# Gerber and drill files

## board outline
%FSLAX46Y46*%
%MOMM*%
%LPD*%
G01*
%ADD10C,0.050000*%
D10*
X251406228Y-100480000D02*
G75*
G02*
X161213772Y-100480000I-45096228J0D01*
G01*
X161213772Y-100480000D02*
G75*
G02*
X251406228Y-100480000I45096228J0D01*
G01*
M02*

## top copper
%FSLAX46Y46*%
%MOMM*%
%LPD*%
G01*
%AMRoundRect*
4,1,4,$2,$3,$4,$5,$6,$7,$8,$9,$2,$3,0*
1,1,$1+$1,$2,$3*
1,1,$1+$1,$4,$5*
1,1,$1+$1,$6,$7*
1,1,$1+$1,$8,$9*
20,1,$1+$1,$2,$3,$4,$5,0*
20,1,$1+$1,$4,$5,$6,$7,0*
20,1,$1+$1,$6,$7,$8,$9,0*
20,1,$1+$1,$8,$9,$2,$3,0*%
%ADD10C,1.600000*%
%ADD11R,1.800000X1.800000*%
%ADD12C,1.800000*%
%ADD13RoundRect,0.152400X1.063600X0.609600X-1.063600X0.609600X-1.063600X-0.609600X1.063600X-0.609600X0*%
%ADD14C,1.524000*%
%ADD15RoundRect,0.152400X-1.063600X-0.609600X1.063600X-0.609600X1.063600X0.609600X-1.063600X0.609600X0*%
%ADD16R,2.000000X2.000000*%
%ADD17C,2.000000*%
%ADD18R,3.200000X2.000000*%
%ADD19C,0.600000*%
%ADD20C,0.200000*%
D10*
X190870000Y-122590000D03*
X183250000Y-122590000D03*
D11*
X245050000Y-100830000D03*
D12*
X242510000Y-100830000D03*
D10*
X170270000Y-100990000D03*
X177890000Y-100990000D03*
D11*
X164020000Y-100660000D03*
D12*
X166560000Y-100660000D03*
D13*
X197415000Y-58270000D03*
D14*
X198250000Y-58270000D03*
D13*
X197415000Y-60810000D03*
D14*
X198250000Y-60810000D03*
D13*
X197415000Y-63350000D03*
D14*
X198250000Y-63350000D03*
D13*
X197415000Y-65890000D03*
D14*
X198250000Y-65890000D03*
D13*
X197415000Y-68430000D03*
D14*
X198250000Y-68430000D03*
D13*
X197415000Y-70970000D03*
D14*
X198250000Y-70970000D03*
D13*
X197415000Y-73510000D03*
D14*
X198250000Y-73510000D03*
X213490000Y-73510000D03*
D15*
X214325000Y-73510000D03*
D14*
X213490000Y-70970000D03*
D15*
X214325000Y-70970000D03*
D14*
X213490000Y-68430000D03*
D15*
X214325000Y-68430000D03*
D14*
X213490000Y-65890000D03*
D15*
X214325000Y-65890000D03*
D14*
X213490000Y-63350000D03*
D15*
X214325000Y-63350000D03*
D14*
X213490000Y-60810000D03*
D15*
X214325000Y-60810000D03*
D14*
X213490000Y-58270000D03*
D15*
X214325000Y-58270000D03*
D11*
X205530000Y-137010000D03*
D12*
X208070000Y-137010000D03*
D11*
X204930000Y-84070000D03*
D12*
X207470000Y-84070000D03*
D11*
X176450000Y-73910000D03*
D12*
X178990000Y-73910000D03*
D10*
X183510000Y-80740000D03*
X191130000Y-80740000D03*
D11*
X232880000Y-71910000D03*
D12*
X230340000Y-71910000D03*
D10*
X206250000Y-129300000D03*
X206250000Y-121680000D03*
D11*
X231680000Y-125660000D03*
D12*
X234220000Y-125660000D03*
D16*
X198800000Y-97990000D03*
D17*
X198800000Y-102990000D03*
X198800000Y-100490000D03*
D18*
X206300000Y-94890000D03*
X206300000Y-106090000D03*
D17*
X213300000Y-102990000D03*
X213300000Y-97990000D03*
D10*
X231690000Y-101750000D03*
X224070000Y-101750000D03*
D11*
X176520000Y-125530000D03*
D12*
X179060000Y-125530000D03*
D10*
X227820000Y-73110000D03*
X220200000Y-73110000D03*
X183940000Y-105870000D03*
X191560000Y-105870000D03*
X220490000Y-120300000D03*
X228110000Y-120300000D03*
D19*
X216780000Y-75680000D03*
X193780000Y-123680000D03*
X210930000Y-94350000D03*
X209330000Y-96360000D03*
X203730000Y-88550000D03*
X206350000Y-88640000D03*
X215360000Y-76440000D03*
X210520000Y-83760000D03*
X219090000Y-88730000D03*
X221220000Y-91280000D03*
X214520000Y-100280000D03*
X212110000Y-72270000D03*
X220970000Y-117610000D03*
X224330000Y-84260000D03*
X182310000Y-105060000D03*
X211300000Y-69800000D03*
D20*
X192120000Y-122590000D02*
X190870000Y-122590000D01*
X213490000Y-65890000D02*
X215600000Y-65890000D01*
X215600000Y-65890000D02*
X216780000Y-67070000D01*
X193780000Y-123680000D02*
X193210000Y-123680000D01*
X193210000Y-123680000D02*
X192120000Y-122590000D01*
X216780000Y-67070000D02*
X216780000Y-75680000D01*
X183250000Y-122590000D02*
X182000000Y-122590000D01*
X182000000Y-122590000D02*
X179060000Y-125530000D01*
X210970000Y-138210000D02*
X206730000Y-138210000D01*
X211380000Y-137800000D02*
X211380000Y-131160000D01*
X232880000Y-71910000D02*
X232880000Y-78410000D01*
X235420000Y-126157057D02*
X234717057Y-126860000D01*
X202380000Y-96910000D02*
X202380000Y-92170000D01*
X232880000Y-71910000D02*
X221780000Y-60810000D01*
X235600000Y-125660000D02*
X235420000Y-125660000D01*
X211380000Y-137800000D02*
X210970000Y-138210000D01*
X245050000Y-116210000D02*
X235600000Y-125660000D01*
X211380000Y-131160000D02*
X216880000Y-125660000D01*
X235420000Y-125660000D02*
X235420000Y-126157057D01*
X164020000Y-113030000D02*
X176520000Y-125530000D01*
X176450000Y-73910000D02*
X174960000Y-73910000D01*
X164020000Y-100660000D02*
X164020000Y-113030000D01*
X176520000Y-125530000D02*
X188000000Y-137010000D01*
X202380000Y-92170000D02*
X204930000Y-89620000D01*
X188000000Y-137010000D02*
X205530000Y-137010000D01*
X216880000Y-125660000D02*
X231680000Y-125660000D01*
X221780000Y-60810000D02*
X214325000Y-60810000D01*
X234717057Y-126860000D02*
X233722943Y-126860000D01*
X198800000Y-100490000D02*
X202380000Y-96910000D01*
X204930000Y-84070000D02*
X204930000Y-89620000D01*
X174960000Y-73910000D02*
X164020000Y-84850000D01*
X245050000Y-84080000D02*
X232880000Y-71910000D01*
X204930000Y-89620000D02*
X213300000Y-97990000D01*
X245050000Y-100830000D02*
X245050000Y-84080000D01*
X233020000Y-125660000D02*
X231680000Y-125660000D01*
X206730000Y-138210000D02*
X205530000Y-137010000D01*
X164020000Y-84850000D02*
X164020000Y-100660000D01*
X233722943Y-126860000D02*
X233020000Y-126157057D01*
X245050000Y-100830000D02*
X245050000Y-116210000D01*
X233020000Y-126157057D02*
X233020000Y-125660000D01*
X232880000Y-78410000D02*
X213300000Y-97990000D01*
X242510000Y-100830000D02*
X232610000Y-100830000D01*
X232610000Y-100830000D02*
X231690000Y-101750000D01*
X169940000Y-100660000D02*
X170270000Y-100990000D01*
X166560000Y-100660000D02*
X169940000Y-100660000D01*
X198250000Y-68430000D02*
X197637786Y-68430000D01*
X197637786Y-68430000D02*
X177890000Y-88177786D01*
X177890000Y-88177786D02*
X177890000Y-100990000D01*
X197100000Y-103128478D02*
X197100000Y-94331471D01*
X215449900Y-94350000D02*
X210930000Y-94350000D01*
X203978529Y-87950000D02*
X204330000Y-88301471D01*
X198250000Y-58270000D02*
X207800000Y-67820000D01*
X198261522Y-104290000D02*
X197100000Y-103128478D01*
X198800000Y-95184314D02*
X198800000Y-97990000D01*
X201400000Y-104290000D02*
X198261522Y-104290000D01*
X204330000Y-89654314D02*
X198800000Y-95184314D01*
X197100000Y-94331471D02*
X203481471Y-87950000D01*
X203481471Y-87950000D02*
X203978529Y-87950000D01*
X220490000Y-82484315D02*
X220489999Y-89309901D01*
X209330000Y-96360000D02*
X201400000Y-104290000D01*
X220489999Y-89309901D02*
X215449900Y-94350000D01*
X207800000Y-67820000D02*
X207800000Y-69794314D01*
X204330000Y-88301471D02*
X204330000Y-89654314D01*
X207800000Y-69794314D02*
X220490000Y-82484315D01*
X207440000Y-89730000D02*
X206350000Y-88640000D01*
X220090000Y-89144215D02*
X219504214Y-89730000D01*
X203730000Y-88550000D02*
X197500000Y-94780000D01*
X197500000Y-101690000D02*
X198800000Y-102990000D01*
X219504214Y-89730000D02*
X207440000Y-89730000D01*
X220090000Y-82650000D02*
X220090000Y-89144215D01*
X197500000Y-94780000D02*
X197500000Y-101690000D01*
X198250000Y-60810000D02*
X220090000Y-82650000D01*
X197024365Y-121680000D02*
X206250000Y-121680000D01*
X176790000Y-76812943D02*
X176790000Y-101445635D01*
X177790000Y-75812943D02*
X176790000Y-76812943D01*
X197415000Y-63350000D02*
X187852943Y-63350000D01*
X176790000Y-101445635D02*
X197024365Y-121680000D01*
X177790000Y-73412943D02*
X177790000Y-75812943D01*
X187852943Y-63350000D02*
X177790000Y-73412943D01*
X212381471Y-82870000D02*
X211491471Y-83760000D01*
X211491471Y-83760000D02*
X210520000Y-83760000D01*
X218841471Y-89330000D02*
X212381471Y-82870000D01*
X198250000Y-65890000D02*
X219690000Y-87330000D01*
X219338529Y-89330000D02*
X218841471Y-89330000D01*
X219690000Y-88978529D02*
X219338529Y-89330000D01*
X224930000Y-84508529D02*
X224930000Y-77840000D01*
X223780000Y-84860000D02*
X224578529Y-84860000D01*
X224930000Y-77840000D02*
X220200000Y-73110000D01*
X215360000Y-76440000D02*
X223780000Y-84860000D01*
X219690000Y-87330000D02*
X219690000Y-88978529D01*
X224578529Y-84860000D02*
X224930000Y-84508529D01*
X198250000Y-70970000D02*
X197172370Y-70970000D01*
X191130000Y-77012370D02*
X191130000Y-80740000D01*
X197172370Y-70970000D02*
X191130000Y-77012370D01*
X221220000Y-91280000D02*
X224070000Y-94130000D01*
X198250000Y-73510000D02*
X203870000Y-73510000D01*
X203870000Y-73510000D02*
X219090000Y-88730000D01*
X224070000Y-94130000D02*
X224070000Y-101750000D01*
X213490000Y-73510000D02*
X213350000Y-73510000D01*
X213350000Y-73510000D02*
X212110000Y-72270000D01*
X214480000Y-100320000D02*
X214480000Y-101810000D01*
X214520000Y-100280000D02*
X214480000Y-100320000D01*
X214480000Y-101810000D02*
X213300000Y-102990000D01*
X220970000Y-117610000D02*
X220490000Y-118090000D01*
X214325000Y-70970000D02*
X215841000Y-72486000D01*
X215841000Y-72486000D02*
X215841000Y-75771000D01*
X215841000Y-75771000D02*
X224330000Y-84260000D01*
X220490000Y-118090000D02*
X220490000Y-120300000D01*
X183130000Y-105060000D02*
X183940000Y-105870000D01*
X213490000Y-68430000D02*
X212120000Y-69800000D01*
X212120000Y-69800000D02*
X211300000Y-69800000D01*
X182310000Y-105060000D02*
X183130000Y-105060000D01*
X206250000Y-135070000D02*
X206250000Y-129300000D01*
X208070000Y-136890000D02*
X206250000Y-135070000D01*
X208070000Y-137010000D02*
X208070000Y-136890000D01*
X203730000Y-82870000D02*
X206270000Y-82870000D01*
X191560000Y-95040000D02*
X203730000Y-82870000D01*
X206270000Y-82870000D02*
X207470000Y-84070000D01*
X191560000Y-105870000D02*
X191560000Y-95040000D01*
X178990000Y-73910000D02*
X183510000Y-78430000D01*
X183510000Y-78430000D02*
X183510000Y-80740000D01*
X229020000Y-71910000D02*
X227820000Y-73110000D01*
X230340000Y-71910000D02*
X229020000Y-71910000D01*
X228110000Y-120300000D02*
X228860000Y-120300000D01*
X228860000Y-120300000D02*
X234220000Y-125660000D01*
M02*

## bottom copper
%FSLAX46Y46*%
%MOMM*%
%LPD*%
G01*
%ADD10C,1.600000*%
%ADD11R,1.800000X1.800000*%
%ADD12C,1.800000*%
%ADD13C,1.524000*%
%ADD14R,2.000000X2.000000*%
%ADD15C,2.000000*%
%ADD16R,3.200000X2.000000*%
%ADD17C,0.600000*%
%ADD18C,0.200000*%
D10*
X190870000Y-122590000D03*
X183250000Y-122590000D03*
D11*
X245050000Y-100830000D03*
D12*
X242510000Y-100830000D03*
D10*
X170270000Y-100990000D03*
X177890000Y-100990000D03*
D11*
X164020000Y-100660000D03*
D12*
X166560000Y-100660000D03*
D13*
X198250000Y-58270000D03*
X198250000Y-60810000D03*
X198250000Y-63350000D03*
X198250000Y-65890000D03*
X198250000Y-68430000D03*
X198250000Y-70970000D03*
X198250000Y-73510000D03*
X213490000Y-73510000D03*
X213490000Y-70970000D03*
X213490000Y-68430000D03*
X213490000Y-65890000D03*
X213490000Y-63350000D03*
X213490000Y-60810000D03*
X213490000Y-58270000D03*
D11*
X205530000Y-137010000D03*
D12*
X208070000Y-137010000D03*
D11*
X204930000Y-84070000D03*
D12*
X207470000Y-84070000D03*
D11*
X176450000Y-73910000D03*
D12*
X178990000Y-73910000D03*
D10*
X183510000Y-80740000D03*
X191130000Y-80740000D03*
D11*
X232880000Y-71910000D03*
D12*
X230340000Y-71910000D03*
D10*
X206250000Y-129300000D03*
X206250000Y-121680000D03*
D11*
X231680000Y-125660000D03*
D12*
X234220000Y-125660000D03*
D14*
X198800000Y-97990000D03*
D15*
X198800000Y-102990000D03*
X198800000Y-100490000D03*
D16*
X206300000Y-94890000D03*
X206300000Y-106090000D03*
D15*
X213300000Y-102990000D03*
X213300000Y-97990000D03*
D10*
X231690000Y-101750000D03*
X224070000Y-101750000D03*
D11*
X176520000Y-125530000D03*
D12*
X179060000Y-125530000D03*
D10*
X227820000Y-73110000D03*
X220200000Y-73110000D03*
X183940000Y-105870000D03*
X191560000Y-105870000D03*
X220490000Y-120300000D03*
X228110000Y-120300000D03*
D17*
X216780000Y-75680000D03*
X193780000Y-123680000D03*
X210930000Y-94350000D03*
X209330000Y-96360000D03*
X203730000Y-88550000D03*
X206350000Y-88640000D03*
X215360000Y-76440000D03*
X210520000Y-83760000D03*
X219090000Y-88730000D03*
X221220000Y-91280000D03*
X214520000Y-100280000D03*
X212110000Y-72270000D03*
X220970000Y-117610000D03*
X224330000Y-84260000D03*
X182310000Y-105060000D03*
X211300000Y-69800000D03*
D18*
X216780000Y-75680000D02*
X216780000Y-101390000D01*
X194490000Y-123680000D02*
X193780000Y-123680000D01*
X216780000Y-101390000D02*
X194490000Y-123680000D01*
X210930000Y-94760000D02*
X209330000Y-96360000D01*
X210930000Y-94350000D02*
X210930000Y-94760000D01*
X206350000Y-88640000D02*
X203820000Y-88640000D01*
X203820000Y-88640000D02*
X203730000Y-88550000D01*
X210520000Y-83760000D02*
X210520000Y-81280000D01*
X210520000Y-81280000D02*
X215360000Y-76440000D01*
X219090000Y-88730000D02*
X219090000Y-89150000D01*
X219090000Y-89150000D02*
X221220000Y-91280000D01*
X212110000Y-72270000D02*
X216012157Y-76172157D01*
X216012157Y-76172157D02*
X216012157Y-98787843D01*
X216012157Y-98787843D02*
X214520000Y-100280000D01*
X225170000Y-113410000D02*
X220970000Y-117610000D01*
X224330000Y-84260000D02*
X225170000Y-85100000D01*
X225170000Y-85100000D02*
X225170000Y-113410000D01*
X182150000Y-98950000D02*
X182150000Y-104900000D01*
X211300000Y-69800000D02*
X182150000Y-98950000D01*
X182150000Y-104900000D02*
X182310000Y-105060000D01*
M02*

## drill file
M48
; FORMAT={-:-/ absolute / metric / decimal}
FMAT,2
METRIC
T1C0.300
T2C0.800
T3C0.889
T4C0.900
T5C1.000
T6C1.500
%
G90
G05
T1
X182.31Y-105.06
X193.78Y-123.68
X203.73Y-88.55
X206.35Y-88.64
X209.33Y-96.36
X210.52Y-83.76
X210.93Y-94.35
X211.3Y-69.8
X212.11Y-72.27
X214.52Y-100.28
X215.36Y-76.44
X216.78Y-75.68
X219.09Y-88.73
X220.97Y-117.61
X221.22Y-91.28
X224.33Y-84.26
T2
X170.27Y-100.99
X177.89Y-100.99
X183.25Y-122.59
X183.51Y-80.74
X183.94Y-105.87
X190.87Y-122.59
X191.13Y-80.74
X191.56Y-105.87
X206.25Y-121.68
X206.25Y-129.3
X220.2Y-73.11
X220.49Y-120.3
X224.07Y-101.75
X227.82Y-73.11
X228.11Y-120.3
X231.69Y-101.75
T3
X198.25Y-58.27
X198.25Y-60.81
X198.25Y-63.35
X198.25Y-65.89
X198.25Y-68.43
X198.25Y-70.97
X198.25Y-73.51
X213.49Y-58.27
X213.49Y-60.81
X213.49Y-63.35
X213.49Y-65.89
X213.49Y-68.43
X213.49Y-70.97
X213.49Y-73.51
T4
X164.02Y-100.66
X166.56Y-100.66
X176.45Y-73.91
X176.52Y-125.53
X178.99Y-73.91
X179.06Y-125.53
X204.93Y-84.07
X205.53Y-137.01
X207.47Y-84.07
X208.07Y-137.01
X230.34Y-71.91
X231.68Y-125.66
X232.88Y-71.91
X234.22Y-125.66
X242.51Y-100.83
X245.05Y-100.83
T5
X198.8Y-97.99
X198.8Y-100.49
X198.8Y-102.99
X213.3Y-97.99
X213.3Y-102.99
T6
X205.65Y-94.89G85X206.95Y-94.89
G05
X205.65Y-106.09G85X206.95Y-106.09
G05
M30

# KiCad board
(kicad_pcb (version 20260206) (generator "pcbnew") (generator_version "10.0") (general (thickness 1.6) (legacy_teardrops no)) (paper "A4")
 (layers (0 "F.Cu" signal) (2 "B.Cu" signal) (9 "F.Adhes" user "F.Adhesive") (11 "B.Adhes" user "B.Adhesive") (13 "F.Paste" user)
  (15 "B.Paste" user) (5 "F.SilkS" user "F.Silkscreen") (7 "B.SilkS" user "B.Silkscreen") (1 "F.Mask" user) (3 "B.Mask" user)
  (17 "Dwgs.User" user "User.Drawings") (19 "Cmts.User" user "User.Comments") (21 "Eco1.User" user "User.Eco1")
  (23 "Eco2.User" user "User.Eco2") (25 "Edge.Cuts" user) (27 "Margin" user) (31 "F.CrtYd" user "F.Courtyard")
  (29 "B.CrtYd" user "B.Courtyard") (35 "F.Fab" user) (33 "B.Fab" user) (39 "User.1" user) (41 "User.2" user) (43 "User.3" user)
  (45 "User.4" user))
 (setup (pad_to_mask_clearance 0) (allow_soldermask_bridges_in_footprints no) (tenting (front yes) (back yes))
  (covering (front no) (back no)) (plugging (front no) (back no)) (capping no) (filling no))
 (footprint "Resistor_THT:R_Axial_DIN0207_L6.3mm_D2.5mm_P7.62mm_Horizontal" (layer "F.Cu") (at 190.87 122.59 180)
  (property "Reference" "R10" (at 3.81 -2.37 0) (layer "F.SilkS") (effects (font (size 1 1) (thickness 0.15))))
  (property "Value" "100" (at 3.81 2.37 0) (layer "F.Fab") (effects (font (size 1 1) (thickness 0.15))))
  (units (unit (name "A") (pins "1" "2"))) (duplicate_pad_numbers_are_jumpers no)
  (pad "1" thru_hole circle (at 0 0 180) (size 1.6 1.6) (drill 0.8) (layers "*.Cu" "*.Mask") (remove_unused_layers no)
   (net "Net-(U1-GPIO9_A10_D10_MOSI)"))
  (pad "2" thru_hole circle (at 7.62 0 180) (size 1.6 1.6) (drill 0.8) (layers "*.Cu" "*.Mask") (remove_unused_layers no) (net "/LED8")))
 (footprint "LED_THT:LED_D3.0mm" (layer "F.Cu") (at 245.05 100.83 180)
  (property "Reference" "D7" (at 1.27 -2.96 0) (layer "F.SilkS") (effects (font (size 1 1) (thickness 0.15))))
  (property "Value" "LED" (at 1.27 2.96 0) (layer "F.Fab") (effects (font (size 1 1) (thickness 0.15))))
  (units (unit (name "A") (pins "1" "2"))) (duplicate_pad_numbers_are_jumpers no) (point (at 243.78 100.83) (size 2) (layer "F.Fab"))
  (pad "1" thru_hole rect (at 0 0 180) (size 1.8 1.8) (drill 0.9) (layers "*.Cu" "*.Mask") (remove_unused_layers no) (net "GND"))
  (pad "2" thru_hole circle (at 2.54 0 180) (size 1.8 1.8) (drill 0.9) (layers "*.Cu" "*.Mask") (remove_unused_layers no) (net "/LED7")))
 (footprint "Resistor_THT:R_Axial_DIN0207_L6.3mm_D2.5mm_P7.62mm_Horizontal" (layer "F.Cu") (at 170.27 100.99)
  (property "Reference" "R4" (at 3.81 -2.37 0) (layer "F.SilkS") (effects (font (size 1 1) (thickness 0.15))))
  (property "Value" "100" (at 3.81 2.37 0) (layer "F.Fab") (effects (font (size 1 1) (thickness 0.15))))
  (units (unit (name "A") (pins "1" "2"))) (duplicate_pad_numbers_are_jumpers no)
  (pad "1" thru_hole circle (at 0 0) (size 1.6 1.6) (drill 0.8) (layers "*.Cu" "*.Mask") (remove_unused_layers no) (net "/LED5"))
  (pad "2" thru_hole circle (at 7.62 0) (size 1.6 1.6) (drill 0.8) (layers "*.Cu" "*.Mask") (remove_unused_layers no)
   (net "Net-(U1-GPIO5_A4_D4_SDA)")))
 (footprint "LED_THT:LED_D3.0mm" (layer "F.Cu") (at 164.02 100.66)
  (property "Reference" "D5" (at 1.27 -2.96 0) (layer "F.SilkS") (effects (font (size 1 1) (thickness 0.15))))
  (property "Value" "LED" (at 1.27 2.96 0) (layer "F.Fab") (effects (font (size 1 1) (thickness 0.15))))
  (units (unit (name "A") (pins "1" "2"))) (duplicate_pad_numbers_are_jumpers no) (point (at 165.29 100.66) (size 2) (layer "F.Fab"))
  (pad "1" thru_hole rect (at 0 0) (size 1.8 1.8) (drill 0.9) (layers "*.Cu" "*.Mask") (remove_unused_layers no) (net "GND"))
  (pad "2" thru_hole circle (at 2.54 0) (size 1.8 1.8) (drill 0.9) (layers "*.Cu" "*.Mask") (remove_unused_layers no) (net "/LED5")))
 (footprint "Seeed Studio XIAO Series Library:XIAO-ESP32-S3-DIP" (layer "F.Cu") (at 205.87 65.89 90)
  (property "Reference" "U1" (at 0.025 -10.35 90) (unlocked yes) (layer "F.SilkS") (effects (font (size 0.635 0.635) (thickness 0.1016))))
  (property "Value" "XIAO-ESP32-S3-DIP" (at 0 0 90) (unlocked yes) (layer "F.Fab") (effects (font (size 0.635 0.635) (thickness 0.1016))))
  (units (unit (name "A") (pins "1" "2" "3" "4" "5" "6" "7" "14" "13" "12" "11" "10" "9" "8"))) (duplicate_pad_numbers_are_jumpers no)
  (pad "1" smd roundrect (at 7.62 -8.455 180) (size 2.432 1.524) (layers "F.Cu" "F.Mask") (roundrect_rratio 0.1) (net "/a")
   (thermal_bridge_angle 45))
  (pad "1" thru_hole circle (at 7.62 -7.62 180) (size 1.524 1.524) (drill 0.889) (layers "*.Cu" "*.Mask") (remove_unused_layers no)
   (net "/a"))
  (pad "2" smd roundrect (at 5.08 -8.455 180) (size 2.432 1.524) (layers "F.Cu" "F.Mask") (roundrect_rratio 0.1) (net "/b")
   (thermal_bridge_angle 45))
  (pad "2" thru_hole circle (at 5.08 -7.62 180) (size 1.524 1.524) (drill 0.889) (layers "*.Cu" "*.Mask") (remove_unused_layers no)
   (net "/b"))
  (pad "3" smd roundrect (at 2.54 -8.455 180) (size 2.432 1.524) (layers "F.Cu" "F.Mask") (roundrect_rratio 0.1)
   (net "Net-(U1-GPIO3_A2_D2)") (thermal_bridge_angle 45))
  (pad "3" thru_hole circle (at 2.54 -7.62 180) (size 1.524 1.524) (drill 0.889) (layers "*.Cu" "*.Mask") (remove_unused_layers no)
   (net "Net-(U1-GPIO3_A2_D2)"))
  (pad "4" smd roundrect (at 0 -8.455 180) (size 2.432 1.524) (layers "F.Cu" "F.Mask") (roundrect_rratio 0.1) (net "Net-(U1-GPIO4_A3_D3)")
   (thermal_bridge_angle 45))
  (pad "4" thru_hole circle (at 0 -7.62 180) (size 1.524 1.524) (drill 0.889) (layers "*.Cu" "*.Mask") (remove_unused_layers no)
   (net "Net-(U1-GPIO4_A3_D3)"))
  (pad "5" smd roundrect (at -2.54 -8.455 180) (size 2.432 1.524) (layers "F.Cu" "F.Mask") (roundrect_rratio 0.1)
   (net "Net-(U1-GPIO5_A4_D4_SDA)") (thermal_bridge_angle 45))
  (pad "5" thru_hole circle (at -2.54 -7.62 180) (size 1.524 1.524) (drill 0.889) (layers "*.Cu" "*.Mask") (remove_unused_layers no)
   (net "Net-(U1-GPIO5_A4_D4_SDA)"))
  (pad "6" smd roundrect (at -5.08 -8.455 180) (size 2.432 1.524) (layers "F.Cu" "F.Mask") (roundrect_rratio 0.1)
   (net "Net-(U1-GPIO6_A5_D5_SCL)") (thermal_bridge_angle 45))
  (pad "6" thru_hole circle (at -5.08 -7.62 180) (size 1.524 1.524) (drill 0.889) (layers "*.Cu" "*.Mask") (remove_unused_layers no)
   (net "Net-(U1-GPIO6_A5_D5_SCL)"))
  (pad "7" smd roundrect (at -7.62 -8.455 180) (size 2.432 1.524) (layers "F.Cu" "F.Mask") (roundrect_rratio 0.1)
   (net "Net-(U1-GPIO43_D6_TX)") (thermal_bridge_angle 45))
  (pad "7" thru_hole circle (at -7.62 -7.62 180) (size 1.524 1.524) (drill 0.889) (layers "*.Cu" "*.Mask") (remove_unused_layers no)
   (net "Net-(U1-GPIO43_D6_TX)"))
  (pad "8" thru_hole circle (at -7.62 7.62) (size 1.524 1.524) (drill 0.889) (layers "*.Cu" "*.Mask") (remove_unused_layers no)
   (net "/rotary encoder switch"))
  (pad "8" smd roundrect (at -7.62 8.455) (size 2.432 1.524) (layers "F.Cu" "F.Mask") (roundrect_rratio 0.1) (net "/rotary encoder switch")
   (thermal_bridge_angle 45))
  (pad "9" thru_hole circle (at -5.08 7.62) (size 1.524 1.524) (drill 0.889) (layers "*.Cu" "*.Mask") (remove_unused_layers no)
   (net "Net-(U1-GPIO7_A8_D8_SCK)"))
  (pad "9" smd roundrect (at -5.08 8.455) (size 2.432 1.524) (layers "F.Cu" "F.Mask") (roundrect_rratio 0.1)
   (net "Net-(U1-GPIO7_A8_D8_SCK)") (thermal_bridge_angle 45))
  (pad "10" thru_hole circle (at -2.54 7.62) (size 1.524 1.524) (drill 0.889) (layers "*.Cu" "*.Mask") (remove_unused_layers no)
   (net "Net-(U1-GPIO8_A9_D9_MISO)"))
  (pad "10" smd roundrect (at -2.54 8.455) (size 2.432 1.524) (layers "F.Cu" "F.Mask") (roundrect_rratio 0.1)
   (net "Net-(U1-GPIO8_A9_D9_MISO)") (thermal_bridge_angle 45))
  (pad "11" thru_hole circle (at 0 7.62) (size 1.524 1.524) (drill 0.889) (layers "*.Cu" "*.Mask") (remove_unused_layers no)
   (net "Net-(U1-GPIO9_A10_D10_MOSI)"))
  (pad "11" smd roundrect (at 0 8.455) (size 2.432 1.524) (layers "F.Cu" "F.Mask") (roundrect_rratio 0.1)
   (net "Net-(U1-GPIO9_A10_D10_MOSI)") (thermal_bridge_angle 45))
  (pad "12" thru_hole circle (at 2.54 7.62) (size 1.524 1.524) (drill 0.889) (layers "*.Cu" "*.Mask") (remove_unused_layers no)
   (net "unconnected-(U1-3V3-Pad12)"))
  (pad "12" smd roundrect (at 2.54 8.455) (size 2.432 1.524) (layers "F.Cu" "F.Mask") (roundrect_rratio 0.1)
   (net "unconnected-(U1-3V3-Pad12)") (thermal_bridge_angle 45))
  (pad "13" thru_hole circle (at 5.08 7.62) (size 1.524 1.524) (drill 0.889) (layers "*.Cu" "*.Mask") (remove_unused_layers no) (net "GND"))
  (pad "13" smd roundrect (at 5.08 8.455) (size 2.432 1.524) (layers "F.Cu" "F.Mask") (roundrect_rratio 0.1) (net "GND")
   (thermal_bridge_angle 45))
  (pad "14" thru_hole circle (at 7.62 7.62) (size 1.524 1.524) (drill 0.889) (layers "*.Cu" "*.Mask") (remove_unused_layers no)
   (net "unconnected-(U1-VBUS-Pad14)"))
  (pad "14" smd roundrect (at 7.62 8.455) (size 2.432 1.524) (layers "F.Cu" "F.Mask") (roundrect_rratio 0.1)
   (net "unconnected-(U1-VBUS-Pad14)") (thermal_bridge_angle 45)))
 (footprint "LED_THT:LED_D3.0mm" (layer "F.Cu") (at 205.53 137.01)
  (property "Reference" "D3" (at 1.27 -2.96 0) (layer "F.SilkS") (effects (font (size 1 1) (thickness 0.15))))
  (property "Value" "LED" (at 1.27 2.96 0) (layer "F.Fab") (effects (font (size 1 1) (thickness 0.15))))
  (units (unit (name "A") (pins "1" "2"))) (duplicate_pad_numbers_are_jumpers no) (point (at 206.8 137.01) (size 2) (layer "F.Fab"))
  (pad "1" thru_hole rect (at 0 0) (size 1.8 1.8) (drill 0.9) (layers "*.Cu" "*.Mask") (remove_unused_layers no) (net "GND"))
  (pad "2" thru_hole circle (at 2.54 0) (size 1.8 1.8) (drill 0.9) (layers "*.Cu" "*.Mask") (remove_unused_layers no) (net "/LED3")))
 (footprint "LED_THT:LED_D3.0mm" (layer "F.Cu") (at 204.93 84.07)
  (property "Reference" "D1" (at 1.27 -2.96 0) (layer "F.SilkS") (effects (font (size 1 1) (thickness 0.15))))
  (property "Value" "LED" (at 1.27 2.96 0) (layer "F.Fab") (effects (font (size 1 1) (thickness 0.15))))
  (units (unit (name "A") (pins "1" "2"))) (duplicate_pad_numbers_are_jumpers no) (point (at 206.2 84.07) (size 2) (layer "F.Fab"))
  (pad "1" thru_hole rect (at 0 0) (size 1.8 1.8) (drill 0.9) (layers "*.Cu" "*.Mask") (remove_unused_layers no) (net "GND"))
  (pad "2" thru_hole circle (at 2.54 0) (size 1.8 1.8) (drill 0.9) (layers "*.Cu" "*.Mask") (remove_unused_layers no) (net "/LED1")))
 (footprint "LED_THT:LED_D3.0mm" (layer "F.Cu") (at 176.45 73.91)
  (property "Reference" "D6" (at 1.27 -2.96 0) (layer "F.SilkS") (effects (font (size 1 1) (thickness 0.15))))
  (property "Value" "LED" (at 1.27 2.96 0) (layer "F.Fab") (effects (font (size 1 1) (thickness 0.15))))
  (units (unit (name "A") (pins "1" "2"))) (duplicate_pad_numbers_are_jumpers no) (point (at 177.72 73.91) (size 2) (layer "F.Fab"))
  (pad "1" thru_hole rect (at 0 0) (size 1.8 1.8) (drill 0.9) (layers "*.Cu" "*.Mask") (remove_unused_layers no) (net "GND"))
  (pad "2" thru_hole circle (at 2.54 0) (size 1.8 1.8) (drill 0.9) (layers "*.Cu" "*.Mask") (remove_unused_layers no) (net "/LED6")))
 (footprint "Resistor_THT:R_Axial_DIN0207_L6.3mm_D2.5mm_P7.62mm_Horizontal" (layer "F.Cu") (at 183.51 80.74)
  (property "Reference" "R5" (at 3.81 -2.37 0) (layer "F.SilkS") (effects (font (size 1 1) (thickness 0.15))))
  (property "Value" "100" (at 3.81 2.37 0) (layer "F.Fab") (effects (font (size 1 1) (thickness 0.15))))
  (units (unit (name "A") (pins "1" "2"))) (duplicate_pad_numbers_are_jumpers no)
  (pad "1" thru_hole circle (at 0 0) (size 1.6 1.6) (drill 0.8) (layers "*.Cu" "*.Mask") (remove_unused_layers no) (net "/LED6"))
  (pad "2" thru_hole circle (at 7.62 0) (size 1.6 1.6) (drill 0.8) (layers "*.Cu" "*.Mask") (remove_unused_layers no)
   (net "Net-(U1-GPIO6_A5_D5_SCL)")))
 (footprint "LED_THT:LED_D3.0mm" (layer "F.Cu") (at 232.88 71.91 180)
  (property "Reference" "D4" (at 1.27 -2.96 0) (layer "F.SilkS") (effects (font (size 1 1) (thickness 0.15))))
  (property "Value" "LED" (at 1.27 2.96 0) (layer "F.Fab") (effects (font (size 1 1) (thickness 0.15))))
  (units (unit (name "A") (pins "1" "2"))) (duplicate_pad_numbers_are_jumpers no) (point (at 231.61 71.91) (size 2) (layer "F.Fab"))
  (pad "1" thru_hole rect (at 0 0 180) (size 1.8 1.8) (drill 0.9) (layers "*.Cu" "*.Mask") (remove_unused_layers no) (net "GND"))
  (pad "2" thru_hole circle (at 2.54 0 180) (size 1.8 1.8) (drill 0.9) (layers "*.Cu" "*.Mask") (remove_unused_layers no) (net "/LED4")))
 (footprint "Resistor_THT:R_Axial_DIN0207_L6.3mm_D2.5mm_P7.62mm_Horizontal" (layer "F.Cu") (at 206.25 129.3 90)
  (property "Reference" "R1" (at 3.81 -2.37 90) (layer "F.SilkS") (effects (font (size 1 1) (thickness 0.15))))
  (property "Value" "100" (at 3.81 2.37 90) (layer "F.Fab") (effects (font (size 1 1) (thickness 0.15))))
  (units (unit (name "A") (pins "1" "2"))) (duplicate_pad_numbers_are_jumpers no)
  (pad "1" thru_hole circle (at 0 0 90) (size 1.6 1.6) (drill 0.8) (layers "*.Cu" "*.Mask") (remove_unused_layers no) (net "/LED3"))
  (pad "2" thru_hole circle (at 7.62 0 90) (size 1.6 1.6) (drill 0.8) (layers "*.Cu" "*.Mask") (remove_unused_layers no)
   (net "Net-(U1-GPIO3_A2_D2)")))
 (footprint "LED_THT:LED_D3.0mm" (layer "F.Cu") (at 231.68 125.66)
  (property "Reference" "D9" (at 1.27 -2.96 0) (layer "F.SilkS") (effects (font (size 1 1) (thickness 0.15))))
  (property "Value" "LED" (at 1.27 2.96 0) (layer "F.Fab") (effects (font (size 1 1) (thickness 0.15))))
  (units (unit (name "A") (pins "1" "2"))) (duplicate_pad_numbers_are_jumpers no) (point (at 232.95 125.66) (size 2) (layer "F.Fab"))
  (pad "1" thru_hole rect (at 0 0) (size 1.8 1.8) (drill 0.9) (layers "*.Cu" "*.Mask") (remove_unused_layers no) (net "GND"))
  (pad "2" thru_hole circle (at 2.54 0) (size 1.8 1.8) (drill 0.9) (layers "*.Cu" "*.Mask") (remove_unused_layers no) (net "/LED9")))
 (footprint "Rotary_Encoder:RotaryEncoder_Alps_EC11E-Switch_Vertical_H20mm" (layer "F.Cu") (at 198.8 97.99)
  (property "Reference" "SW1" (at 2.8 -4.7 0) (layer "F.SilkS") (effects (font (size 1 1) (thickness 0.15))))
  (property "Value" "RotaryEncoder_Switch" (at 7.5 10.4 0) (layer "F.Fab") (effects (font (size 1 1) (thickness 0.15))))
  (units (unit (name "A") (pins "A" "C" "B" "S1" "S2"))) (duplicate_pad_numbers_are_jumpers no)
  (pad "A" thru_hole rect (at 0 0) (size 2 2) (drill 1) (layers "*.Cu" "*.Mask") (remove_unused_layers no) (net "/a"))
  (pad "B" thru_hole circle (at 0 5) (size 2 2) (drill 1) (layers "*.Cu" "*.Mask") (remove_unused_layers no) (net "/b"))
  (pad "C" thru_hole circle (at 0 2.5) (size 2 2) (drill 1) (layers "*.Cu" "*.Mask") (remove_unused_layers no) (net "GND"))
  (pad "MP" thru_hole rect (at 7.5 -3.1) (size 3.2 2) (drill oval 2.8 1.5) (layers "*.Cu" "*.Mask") (remove_unused_layers no))
  (pad "MP" thru_hole rect (at 7.5 8.1) (size 3.2 2) (drill oval 2.8 1.5) (layers "*.Cu" "*.Mask") (remove_unused_layers no))
  (pad "S1" thru_hole circle (at 14.5 5) (size 2 2) (drill 1) (layers "*.Cu" "*.Mask") (remove_unused_layers no)
   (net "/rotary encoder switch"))
  (pad "S2" thru_hole circle (at 14.5 0) (size 2 2) (drill 1) (layers "*.Cu" "*.Mask") (remove_unused_layers no) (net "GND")))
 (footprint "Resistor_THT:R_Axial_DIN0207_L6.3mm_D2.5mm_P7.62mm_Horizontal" (layer "F.Cu") (at 231.69 101.75 180)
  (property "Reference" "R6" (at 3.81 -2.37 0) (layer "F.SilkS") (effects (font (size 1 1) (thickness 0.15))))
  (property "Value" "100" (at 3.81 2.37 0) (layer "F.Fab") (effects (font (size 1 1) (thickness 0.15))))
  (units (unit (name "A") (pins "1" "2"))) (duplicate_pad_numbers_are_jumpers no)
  (pad "1" thru_hole circle (at 0 0 180) (size 1.6 1.6) (drill 0.8) (layers "*.Cu" "*.Mask") (remove_unused_layers no) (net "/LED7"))
  (pad "2" thru_hole circle (at 7.62 0 180) (size 1.6 1.6) (drill 0.8) (layers "*.Cu" "*.Mask") (remove_unused_layers no)
   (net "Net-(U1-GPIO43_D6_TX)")))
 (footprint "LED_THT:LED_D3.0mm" (layer "F.Cu") (at 176.52 125.53)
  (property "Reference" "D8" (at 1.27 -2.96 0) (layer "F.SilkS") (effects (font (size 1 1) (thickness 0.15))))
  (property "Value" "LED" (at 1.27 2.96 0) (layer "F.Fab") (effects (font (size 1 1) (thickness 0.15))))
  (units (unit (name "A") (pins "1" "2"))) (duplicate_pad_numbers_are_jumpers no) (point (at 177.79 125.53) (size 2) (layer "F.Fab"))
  (pad "1" thru_hole rect (at 0 0) (size 1.8 1.8) (drill 0.9) (layers "*.Cu" "*.Mask") (remove_unused_layers no) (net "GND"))
  (pad "2" thru_hole circle (at 2.54 0) (size 1.8 1.8) (drill 0.9) (layers "*.Cu" "*.Mask") (remove_unused_layers no) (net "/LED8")))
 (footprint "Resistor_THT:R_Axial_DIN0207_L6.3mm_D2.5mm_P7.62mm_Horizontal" (layer "F.Cu") (at 227.82 73.11 180)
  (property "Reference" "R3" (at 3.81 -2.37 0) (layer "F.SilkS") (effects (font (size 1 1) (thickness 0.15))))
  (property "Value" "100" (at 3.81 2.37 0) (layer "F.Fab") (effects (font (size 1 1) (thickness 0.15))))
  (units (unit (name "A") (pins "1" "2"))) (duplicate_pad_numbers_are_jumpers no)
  (pad "1" thru_hole circle (at 0 0 180) (size 1.6 1.6) (drill 0.8) (layers "*.Cu" "*.Mask") (remove_unused_layers no) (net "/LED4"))
  (pad "2" thru_hole circle (at 7.62 0 180) (size 1.6 1.6) (drill 0.8) (layers "*.Cu" "*.Mask") (remove_unused_layers no)
   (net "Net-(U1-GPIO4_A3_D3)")))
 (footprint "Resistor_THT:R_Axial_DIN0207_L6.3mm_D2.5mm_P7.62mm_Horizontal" (layer "F.Cu") (at 183.94 105.87)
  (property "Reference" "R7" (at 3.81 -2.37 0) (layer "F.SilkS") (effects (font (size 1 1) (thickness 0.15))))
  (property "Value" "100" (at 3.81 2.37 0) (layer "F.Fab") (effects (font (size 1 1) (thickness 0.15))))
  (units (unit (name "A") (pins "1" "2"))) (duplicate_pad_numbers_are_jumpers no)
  (pad "1" thru_hole circle (at 0 0) (size 1.6 1.6) (drill 0.8) (layers "*.Cu" "*.Mask") (remove_unused_layers no)
   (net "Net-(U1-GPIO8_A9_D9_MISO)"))
  (pad "2" thru_hole circle (at 7.62 0) (size 1.6 1.6) (drill 0.8) (layers "*.Cu" "*.Mask") (remove_unused_layers no) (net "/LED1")))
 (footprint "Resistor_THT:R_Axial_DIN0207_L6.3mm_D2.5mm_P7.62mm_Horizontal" (layer "F.Cu") (at 220.49 120.3)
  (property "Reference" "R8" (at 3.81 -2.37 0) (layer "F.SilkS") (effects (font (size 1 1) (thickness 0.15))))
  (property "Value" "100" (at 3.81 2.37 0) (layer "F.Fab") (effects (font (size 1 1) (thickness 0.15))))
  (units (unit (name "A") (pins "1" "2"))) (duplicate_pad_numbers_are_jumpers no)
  (pad "1" thru_hole circle (at 0 0) (size 1.6 1.6) (drill 0.8) (layers "*.Cu" "*.Mask") (remove_unused_layers no)
   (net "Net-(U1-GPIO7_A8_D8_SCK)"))
  (pad "2" thru_hole circle (at 7.62 0) (size 1.6 1.6) (drill 0.8) (layers "*.Cu" "*.Mask") (remove_unused_layers no) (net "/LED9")))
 (gr_circle (center 206.31 100.48) (end 244.28 124.81) (stroke (width 0.05) (type default)) (fill no) (layer "Edge.Cuts"))
 (segment (start 192.12 122.59) (end 190.87 122.59) (width 0.2) (layer "F.Cu") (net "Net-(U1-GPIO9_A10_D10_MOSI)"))
 (segment (start 213.49 65.89) (end 215.6 65.89) (width 0.2) (layer "F.Cu") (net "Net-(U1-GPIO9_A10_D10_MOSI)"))
 (segment (start 215.6 65.89) (end 216.78 67.07) (width 0.2) (layer "F.Cu") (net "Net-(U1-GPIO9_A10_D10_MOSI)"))
 (segment (start 193.78 123.68) (end 193.21 123.68) (width 0.2) (layer "F.Cu") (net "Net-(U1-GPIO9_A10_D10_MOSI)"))
 (segment (start 193.21 123.68) (end 192.12 122.59) (width 0.2) (layer "F.Cu") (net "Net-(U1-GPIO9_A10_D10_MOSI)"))
 (segment (start 216.78 67.07) (end 216.78 75.68) (width 0.2) (layer "F.Cu") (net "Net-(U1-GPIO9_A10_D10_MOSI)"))
 (via (at 216.78 75.68) (size 0.6) (drill 0.3) (layers "F.Cu" "B.Cu") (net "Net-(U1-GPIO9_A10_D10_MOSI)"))
 (via (at 193.78 123.68) (size 0.6) (drill 0.3) (layers "F.Cu" "B.Cu") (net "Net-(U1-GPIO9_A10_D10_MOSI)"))
 (segment (start 216.78 75.68) (end 216.78 101.39) (width 0.2) (layer "B.Cu") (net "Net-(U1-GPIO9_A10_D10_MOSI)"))
 (segment (start 194.49 123.68) (end 193.78 123.68) (width 0.2) (layer "B.Cu") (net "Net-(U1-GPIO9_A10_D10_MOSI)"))
 (segment (start 216.78 101.39) (end 194.49 123.68) (width 0.2) (layer "B.Cu") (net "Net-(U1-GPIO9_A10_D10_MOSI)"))
 (segment (start 183.25 122.59) (end 182 122.59) (width 0.2) (layer "F.Cu") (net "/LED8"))
 (segment (start 182 122.59) (end 179.06 125.53) (width 0.2) (layer "F.Cu") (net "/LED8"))
 (segment (start 210.97 138.21) (end 206.73 138.21) (width 0.2) (layer "F.Cu") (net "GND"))
 (segment (start 211.38 137.8) (end 211.38 131.16) (width 0.2) (layer "F.Cu") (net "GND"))
 (segment (start 232.88 71.91) (end 232.88 78.41) (width 0.2) (layer "F.Cu") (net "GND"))
 (segment (start 235.42 126.157057) (end 234.717057 126.86) (width 0.2) (layer "F.Cu") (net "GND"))
 (segment (start 202.38 96.91) (end 202.38 92.17) (width 0.2) (layer "F.Cu") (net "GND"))
 (segment (start 232.88 71.91) (end 221.78 60.81) (width 0.2) (layer "F.Cu") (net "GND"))
 (segment (start 235.6 125.66) (end 235.42 125.66) (width 0.2) (layer "F.Cu") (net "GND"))
 (segment (start 211.38 137.8) (end 210.97 138.21) (width 0.2) (layer "F.Cu") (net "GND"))
 (segment (start 245.05 116.21) (end 235.6 125.66) (width 0.2) (layer "F.Cu") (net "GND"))
 (segment (start 211.38 131.16) (end 216.88 125.66) (width 0.2) (layer "F.Cu") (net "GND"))
 (segment (start 235.42 125.66) (end 235.42 126.157057) (width 0.2) (layer "F.Cu") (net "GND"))
 (segment (start 164.02 113.03) (end 176.52 125.53) (width 0.2) (layer "F.Cu") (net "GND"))
 (segment (start 176.45 73.91) (end 174.96 73.91) (width 0.2) (layer "F.Cu") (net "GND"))
 (segment (start 164.02 100.66) (end 164.02 113.03) (width 0.2) (layer "F.Cu") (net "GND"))
 (segment (start 176.52 125.53) (end 188 137.01) (width 0.2) (layer "F.Cu") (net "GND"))
 (segment (start 202.38 92.17) (end 204.93 89.62) (width 0.2) (layer "F.Cu") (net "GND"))
 (segment (start 188 137.01) (end 205.53 137.01) (width 0.2) (layer "F.Cu") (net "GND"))
 (segment (start 216.88 125.66) (end 231.68 125.66) (width 0.2) (layer "F.Cu") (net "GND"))
 (segment (start 221.78 60.81) (end 214.325 60.81) (width 0.2) (layer "F.Cu") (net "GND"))
 (segment (start 234.717057 126.86) (end 233.722943 126.86) (width 0.2) (layer "F.Cu") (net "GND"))
 (segment (start 198.8 100.49) (end 202.38 96.91) (width 0.2) (layer "F.Cu") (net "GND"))
 (segment (start 204.93 84.07) (end 204.93 89.62) (width 0.2) (layer "F.Cu") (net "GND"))
 (segment (start 174.96 73.91) (end 164.02 84.85) (width 0.2) (layer "F.Cu") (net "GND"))
 (segment (start 245.05 84.08) (end 232.88 71.91) (width 0.2) (layer "F.Cu") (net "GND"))
 (segment (start 204.93 89.62) (end 213.3 97.99) (width 0.2) (layer "F.Cu") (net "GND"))
 (segment (start 245.05 100.83) (end 245.05 84.08) (width 0.2) (layer "F.Cu") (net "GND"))
 (segment (start 233.02 125.66) (end 231.68 125.66) (width 0.2) (layer "F.Cu") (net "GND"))
 (segment (start 206.73 138.21) (end 205.53 137.01) (width 0.2) (layer "F.Cu") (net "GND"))
 (segment (start 164.02 84.85) (end 164.02 100.66) (width 0.2) (layer "F.Cu") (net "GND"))
 (segment (start 233.722943 126.86) (end 233.02 126.157057) (width 0.2) (layer "F.Cu") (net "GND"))
 (segment (start 245.05 100.83) (end 245.05 116.21) (width 0.2) (layer "F.Cu") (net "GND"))
 (segment (start 233.02 126.157057) (end 233.02 125.66) (width 0.2) (layer "F.Cu") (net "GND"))
 (segment (start 232.88 78.41) (end 213.3 97.99) (width 0.2) (layer "F.Cu") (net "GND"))
 (segment (start 242.51 100.83) (end 232.61 100.83) (width 0.2) (layer "F.Cu") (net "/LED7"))
 (segment (start 232.61 100.83) (end 231.69 101.75) (width 0.2) (layer "F.Cu") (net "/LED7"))
 (segment (start 169.94 100.66) (end 170.27 100.99) (width 0.2) (layer "F.Cu") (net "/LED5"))
 (segment (start 166.56 100.66) (end 169.94 100.66) (width 0.2) (layer "F.Cu") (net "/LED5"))
 (segment (start 198.25 68.43) (end 197.637786 68.43) (width 0.2) (layer "F.Cu") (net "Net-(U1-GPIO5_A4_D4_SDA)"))
 (segment (start 197.637786 68.43) (end 177.89 88.177786) (width 0.2) (layer "F.Cu") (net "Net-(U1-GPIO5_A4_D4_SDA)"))
 (segment (start 177.89 88.177786) (end 177.89 100.99) (width 0.2) (layer "F.Cu") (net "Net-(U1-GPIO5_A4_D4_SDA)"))
 (segment (start 197.1 103.128478) (end 197.1 94.331471) (width 0.2) (layer "F.Cu") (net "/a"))
 (segment (start 215.4499 94.35) (end 210.93 94.35) (width 0.2) (layer "F.Cu") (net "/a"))
 (segment (start 203.978529 87.95) (end 204.33 88.301471) (width 0.2) (layer "F.Cu") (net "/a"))
 (segment (start 198.25 58.27) (end 207.8 67.82) (width 0.2) (layer "F.Cu") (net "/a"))
 (segment (start 198.261522 104.29) (end 197.1 103.128478) (width 0.2) (layer "F.Cu") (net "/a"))
 (segment (start 198.8 95.184314) (end 198.8 97.99) (width 0.2) (layer "F.Cu") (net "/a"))
 (segment (start 201.4 104.29) (end 198.261522 104.29) (width 0.2) (layer "F.Cu") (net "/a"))
 (segment (start 204.33 89.654314) (end 198.8 95.184314) (width 0.2) (layer "F.Cu") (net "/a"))
 (segment (start 197.1 94.331471) (end 203.481471 87.95) (width 0.2) (layer "F.Cu") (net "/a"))
 (segment (start 203.481471 87.95) (end 203.978529 87.95) (width 0.2) (layer "F.Cu") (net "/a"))
 (segment (start 220.49 82.484315) (end 220.489999 89.309901) (width 0.2) (layer "F.Cu") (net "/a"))
 (segment (start 209.33 96.36) (end 201.4 104.29) (width 0.2) (layer "F.Cu") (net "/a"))
 (segment (start 220.489999 89.309901) (end 215.4499 94.35) (width 0.2) (layer "F.Cu") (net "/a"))
 (segment (start 207.8 67.82) (end 207.8 69.794314) (width 0.2) (layer "F.Cu") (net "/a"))
 (segment (start 204.33 88.301471) (end 204.33 89.654314) (width 0.2) (layer "F.Cu") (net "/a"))
 (segment (start 207.8 69.794314) (end 220.49 82.484315) (width 0.2) (layer "F.Cu") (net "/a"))
 (via (at 210.93 94.35) (size 0.6) (drill 0.3) (layers "F.Cu" "B.Cu") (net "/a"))
 (via (at 209.33 96.36) (size 0.6) (drill 0.3) (layers "F.Cu" "B.Cu") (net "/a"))
 (segment (start 210.93 94.76) (end 209.33 96.36) (width 0.2) (layer "B.Cu") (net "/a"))
 (segment (start 210.93 94.35) (end 210.93 94.76) (width 0.2) (layer "B.Cu") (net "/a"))
 (segment (start 207.44 89.73) (end 206.35 88.64) (width 0.2) (layer "F.Cu") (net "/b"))
 (segment (start 220.09 89.144215) (end 219.504214 89.73) (width 0.2) (layer "F.Cu") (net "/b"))
 (segment (start 203.73 88.55) (end 197.5 94.78) (width 0.2) (layer "F.Cu") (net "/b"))
 (segment (start 197.5 101.69) (end 198.8 102.99) (width 0.2) (layer "F.Cu") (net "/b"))
 (segment (start 219.504214 89.73) (end 207.44 89.73) (width 0.2) (layer "F.Cu") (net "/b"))
 (segment (start 220.09 82.65) (end 220.09 89.144215) (width 0.2) (layer "F.Cu") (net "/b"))
 (segment (start 197.5 94.78) (end 197.5 101.69) (width 0.2) (layer "F.Cu") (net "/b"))
 (segment (start 198.25 60.81) (end 220.09 82.65) (width 0.2) (layer "F.Cu") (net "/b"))
 (via (at 203.73 88.55) (size 0.6) (drill 0.3) (layers "F.Cu" "B.Cu") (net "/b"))
 (via (at 206.35 88.64) (size 0.6) (drill 0.3) (layers "F.Cu" "B.Cu") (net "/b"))
 (segment (start 206.35 88.64) (end 203.82 88.64) (width 0.2) (layer "B.Cu") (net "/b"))
 (segment (start 203.82 88.64) (end 203.73 88.55) (width 0.2) (layer "B.Cu") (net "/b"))
 (segment (start 197.024365 121.68) (end 206.25 121.68) (width 0.2) (layer "F.Cu") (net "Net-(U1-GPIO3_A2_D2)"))
 (segment (start 176.79 76.812943) (end 176.79 101.445635) (width 0.2) (layer "F.Cu") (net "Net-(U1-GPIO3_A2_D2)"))
 (segment (start 177.79 75.812943) (end 176.79 76.812943) (width 0.2) (layer "F.Cu") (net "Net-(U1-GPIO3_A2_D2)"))
 (segment (start 197.415 63.35) (end 187.852943 63.35) (width 0.2) (layer "F.Cu") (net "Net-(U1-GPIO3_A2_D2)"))
 (segment (start 176.79 101.445635) (end 197.024365 121.68) (width 0.2) (layer "F.Cu") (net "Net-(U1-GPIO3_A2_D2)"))
 (segment (start 177.79 73.412943) (end 177.79 75.812943) (width 0.2) (layer "F.Cu") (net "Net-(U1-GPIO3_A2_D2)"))
 (segment (start 187.852943 63.35) (end 177.79 73.412943) (width 0.2) (layer "F.Cu") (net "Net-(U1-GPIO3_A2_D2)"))
 (segment (start 212.381471 82.87) (end 211.491471 83.76) (width 0.2) (layer "F.Cu") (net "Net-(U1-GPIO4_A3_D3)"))
 (segment (start 211.491471 83.76) (end 210.52 83.76) (width 0.2) (layer "F.Cu") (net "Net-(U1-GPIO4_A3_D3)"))
 (segment (start 218.841471 89.33) (end 212.381471 82.87) (width 0.2) (layer "F.Cu") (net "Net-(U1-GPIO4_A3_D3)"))
 (segment (start 198.25 65.89) (end 219.69 87.33) (width 0.2) (layer "F.Cu") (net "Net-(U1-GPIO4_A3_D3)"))
 (segment (start 219.338529 89.33) (end 218.841471 89.33) (width 0.2) (layer "F.Cu") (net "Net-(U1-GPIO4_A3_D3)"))
 (segment (start 219.69 88.978529) (end 219.338529 89.33) (width 0.2) (layer "F.Cu") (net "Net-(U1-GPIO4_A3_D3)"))
 (segment (start 224.93 84.508529) (end 224.93 77.84) (width 0.2) (layer "F.Cu") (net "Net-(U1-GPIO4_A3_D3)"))
 (segment (start 223.78 84.86) (end 224.578529 84.86) (width 0.2) (layer "F.Cu") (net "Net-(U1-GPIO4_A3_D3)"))
 (segment (start 224.93 77.84) (end 220.2 73.11) (width 0.2) (layer "F.Cu") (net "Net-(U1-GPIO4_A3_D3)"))
 (segment (start 215.36 76.44) (end 223.78 84.86) (width 0.2) (layer "F.Cu") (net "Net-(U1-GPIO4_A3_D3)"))
 (segment (start 219.69 87.33) (end 219.69 88.978529) (width 0.2) (layer "F.Cu") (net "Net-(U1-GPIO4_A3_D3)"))
 (segment (start 224.578529 84.86) (end 224.93 84.508529) (width 0.2) (layer "F.Cu") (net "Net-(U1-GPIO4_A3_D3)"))
 (via (at 215.36 76.44) (size 0.6) (drill 0.3) (layers "F.Cu" "B.Cu") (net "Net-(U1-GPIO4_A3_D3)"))
 (via (at 210.52 83.76) (size 0.6) (drill 0.3) (layers "F.Cu" "B.Cu") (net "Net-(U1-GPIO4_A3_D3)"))
 (segment (start 210.52 83.76) (end 210.52 81.28) (width 0.2) (layer "B.Cu") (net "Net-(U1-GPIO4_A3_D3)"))
 (segment (start 210.52 81.28) (end 215.36 76.44) (width 0.2) (layer "B.Cu") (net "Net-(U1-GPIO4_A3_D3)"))
 (segment (start 198.25 70.97) (end 197.17237 70.97) (width 0.2) (layer "F.Cu") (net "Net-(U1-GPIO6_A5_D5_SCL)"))
 (segment (start 191.13 77.01237) (end 191.13 80.74) (width 0.2) (layer "F.Cu") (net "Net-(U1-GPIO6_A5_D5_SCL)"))
 (segment (start 197.17237 70.97) (end 191.13 77.01237) (width 0.2) (layer "F.Cu") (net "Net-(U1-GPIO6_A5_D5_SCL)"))
 (segment (start 221.22 91.28) (end 224.07 94.13) (width 0.2) (layer "F.Cu") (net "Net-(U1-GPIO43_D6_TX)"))
 (segment (start 198.25 73.51) (end 203.87 73.51) (width 0.2) (layer "F.Cu") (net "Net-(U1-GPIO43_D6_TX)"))
 (segment (start 203.87 73.51) (end 219.09 88.73) (width 0.2) (layer "F.Cu") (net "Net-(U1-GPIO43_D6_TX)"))
 (segment (start 224.07 94.13) (end 224.07 101.75) (width 0.2) (layer "F.Cu") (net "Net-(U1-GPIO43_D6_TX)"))
 (via (at 219.09 88.73) (size 0.6) (drill 0.3) (layers "F.Cu" "B.Cu") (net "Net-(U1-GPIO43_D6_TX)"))
 (via (at 221.22 91.28) (size 0.6) (drill 0.3) (layers "F.Cu" "B.Cu") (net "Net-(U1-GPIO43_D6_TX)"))
 (segment (start 219.09 88.73) (end 219.09 89.15) (width 0.2) (layer "B.Cu") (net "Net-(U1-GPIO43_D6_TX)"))
 (segment (start 219.09 89.15) (end 221.22 91.28) (width 0.2) (layer "B.Cu") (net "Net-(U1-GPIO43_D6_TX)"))
 (segment (start 213.49 73.51) (end 213.35 73.51) (width 0.2) (layer "F.Cu") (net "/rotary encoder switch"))
 (segment (start 213.35 73.51) (end 212.11 72.27) (width 0.2) (layer "F.Cu") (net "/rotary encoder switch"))
 (segment (start 214.48 100.32) (end 214.48 101.81) (width 0.2) (layer "F.Cu") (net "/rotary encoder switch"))
 (segment (start 214.52 100.28) (end 214.48 100.32) (width 0.2) (layer "F.Cu") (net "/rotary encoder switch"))
 (segment (start 214.48 101.81) (end 213.3 102.99) (width 0.2) (layer "F.Cu") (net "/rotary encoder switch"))
 (via (at 214.52 100.28) (size 0.6) (drill 0.3) (layers "F.Cu" "B.Cu") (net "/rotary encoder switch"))
 (via (at 212.11 72.27) (size 0.6) (drill 0.3) (layers "F.Cu" "B.Cu") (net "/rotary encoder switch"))
 (segment (start 212.11 72.27) (end 216.012157 76.172157) (width 0.2) (layer "B.Cu") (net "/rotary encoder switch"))
 (segment (start 216.012157 76.172157) (end 216.012157 98.787843) (width 0.2) (layer "B.Cu") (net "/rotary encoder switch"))
 (segment (start 216.012157 98.787843) (end 214.52 100.28) (width 0.2) (layer "B.Cu") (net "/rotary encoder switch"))
 (segment (start 220.97 117.61) (end 220.49 118.09) (width 0.2) (layer "F.Cu") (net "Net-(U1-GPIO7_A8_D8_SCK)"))
 (segment (start 214.325 70.97) (end 215.841 72.486) (width 0.2) (layer "F.Cu") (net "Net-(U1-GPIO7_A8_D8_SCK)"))
 (segment (start 215.841 72.486) (end 215.841 75.771) (width 0.2) (layer "F.Cu") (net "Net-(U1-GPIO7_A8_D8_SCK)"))
 (segment (start 215.841 75.771) (end 224.33 84.26) (width 0.2) (layer "F.Cu") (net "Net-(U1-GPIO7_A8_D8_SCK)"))
 (segment (start 220.49 118.09) (end 220.49 120.3) (width 0.2) (layer "F.Cu") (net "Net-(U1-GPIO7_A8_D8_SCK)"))
 (via (at 220.97 117.61) (size 0.6) (drill 0.3) (layers "F.Cu" "B.Cu") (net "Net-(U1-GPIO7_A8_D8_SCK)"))
 (via (at 224.33 84.26) (size 0.6) (drill 0.3) (layers "F.Cu" "B.Cu") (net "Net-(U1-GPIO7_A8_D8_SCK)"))
 (segment (start 225.17 113.41) (end 220.97 117.61) (width 0.2) (layer "B.Cu") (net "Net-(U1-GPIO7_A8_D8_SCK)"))
 (segment (start 224.33 84.26) (end 225.17 85.1) (width 0.2) (layer "B.Cu") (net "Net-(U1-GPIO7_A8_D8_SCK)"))
 (segment (start 225.17 85.1) (end 225.17 113.41) (width 0.2) (layer "B.Cu") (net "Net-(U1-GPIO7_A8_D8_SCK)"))
 (segment (start 183.13 105.06) (end 183.94 105.87) (width 0.2) (layer "F.Cu") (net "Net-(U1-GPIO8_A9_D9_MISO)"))
 (segment (start 213.49 68.43) (end 212.12 69.8) (width 0.2) (layer "F.Cu") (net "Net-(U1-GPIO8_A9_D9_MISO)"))
 (segment (start 212.12 69.8) (end 211.3 69.8) (width 0.2) (layer "F.Cu") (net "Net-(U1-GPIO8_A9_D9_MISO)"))
 (segment (start 182.31 105.06) (end 183.13 105.06) (width 0.2) (layer "F.Cu") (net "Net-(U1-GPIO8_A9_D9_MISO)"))
 (via (at 182.31 105.06) (size 0.6) (drill 0.3) (layers "F.Cu" "B.Cu") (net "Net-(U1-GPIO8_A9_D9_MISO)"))
 (via (at 211.3 69.8) (size 0.6) (drill 0.3) (layers "F.Cu" "B.Cu") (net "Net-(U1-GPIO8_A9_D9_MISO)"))
 (segment (start 182.15 98.95) (end 182.15 104.9) (width 0.2) (layer "B.Cu") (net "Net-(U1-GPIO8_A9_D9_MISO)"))
 (segment (start 211.3 69.8) (end 182.15 98.95) (width 0.2) (layer "B.Cu") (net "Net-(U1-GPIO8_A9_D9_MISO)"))
 (segment (start 182.15 104.9) (end 182.31 105.06) (width 0.2) (layer "B.Cu") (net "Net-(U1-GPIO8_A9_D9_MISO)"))
 (segment (start 206.25 135.07) (end 206.25 129.3) (width 0.2) (layer "F.Cu") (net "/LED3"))
 (segment (start 208.07 136.89) (end 206.25 135.07) (width 0.2) (layer "F.Cu") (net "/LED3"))
 (segment (start 208.07 137.01) (end 208.07 136.89) (width 0.2) (layer "F.Cu") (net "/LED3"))
 (segment (start 203.73 82.87) (end 206.27 82.87) (width 0.2) (layer "F.Cu") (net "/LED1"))
 (segment (start 191.56 95.04) (end 203.73 82.87) (width 0.2) (layer "F.Cu") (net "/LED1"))
 (segment (start 206.27 82.87) (end 207.47 84.07) (width 0.2) (layer "F.Cu") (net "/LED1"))
 (segment (start 191.56 105.87) (end 191.56 95.04) (width 0.2) (layer "F.Cu") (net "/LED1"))
 (segment (start 178.99 73.91) (end 183.51 78.43) (width 0.2) (layer "F.Cu") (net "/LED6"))
 (segment (start 183.51 78.43) (end 183.51 80.74) (width 0.2) (layer "F.Cu") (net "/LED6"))
 (segment (start 229.02 71.91) (end 227.82 73.11) (width 0.2) (layer "F.Cu") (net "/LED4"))
 (segment (start 230.34 71.91) (end 229.02 71.91) (width 0.2) (layer "F.Cu") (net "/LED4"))
 (segment (start 228.11 120.3) (end 228.86 120.3) (width 0.2) (layer "F.Cu") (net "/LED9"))
 (segment (start 228.86 120.3) (end 234.22 125.66) (width 0.2) (layer "F.Cu") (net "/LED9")))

